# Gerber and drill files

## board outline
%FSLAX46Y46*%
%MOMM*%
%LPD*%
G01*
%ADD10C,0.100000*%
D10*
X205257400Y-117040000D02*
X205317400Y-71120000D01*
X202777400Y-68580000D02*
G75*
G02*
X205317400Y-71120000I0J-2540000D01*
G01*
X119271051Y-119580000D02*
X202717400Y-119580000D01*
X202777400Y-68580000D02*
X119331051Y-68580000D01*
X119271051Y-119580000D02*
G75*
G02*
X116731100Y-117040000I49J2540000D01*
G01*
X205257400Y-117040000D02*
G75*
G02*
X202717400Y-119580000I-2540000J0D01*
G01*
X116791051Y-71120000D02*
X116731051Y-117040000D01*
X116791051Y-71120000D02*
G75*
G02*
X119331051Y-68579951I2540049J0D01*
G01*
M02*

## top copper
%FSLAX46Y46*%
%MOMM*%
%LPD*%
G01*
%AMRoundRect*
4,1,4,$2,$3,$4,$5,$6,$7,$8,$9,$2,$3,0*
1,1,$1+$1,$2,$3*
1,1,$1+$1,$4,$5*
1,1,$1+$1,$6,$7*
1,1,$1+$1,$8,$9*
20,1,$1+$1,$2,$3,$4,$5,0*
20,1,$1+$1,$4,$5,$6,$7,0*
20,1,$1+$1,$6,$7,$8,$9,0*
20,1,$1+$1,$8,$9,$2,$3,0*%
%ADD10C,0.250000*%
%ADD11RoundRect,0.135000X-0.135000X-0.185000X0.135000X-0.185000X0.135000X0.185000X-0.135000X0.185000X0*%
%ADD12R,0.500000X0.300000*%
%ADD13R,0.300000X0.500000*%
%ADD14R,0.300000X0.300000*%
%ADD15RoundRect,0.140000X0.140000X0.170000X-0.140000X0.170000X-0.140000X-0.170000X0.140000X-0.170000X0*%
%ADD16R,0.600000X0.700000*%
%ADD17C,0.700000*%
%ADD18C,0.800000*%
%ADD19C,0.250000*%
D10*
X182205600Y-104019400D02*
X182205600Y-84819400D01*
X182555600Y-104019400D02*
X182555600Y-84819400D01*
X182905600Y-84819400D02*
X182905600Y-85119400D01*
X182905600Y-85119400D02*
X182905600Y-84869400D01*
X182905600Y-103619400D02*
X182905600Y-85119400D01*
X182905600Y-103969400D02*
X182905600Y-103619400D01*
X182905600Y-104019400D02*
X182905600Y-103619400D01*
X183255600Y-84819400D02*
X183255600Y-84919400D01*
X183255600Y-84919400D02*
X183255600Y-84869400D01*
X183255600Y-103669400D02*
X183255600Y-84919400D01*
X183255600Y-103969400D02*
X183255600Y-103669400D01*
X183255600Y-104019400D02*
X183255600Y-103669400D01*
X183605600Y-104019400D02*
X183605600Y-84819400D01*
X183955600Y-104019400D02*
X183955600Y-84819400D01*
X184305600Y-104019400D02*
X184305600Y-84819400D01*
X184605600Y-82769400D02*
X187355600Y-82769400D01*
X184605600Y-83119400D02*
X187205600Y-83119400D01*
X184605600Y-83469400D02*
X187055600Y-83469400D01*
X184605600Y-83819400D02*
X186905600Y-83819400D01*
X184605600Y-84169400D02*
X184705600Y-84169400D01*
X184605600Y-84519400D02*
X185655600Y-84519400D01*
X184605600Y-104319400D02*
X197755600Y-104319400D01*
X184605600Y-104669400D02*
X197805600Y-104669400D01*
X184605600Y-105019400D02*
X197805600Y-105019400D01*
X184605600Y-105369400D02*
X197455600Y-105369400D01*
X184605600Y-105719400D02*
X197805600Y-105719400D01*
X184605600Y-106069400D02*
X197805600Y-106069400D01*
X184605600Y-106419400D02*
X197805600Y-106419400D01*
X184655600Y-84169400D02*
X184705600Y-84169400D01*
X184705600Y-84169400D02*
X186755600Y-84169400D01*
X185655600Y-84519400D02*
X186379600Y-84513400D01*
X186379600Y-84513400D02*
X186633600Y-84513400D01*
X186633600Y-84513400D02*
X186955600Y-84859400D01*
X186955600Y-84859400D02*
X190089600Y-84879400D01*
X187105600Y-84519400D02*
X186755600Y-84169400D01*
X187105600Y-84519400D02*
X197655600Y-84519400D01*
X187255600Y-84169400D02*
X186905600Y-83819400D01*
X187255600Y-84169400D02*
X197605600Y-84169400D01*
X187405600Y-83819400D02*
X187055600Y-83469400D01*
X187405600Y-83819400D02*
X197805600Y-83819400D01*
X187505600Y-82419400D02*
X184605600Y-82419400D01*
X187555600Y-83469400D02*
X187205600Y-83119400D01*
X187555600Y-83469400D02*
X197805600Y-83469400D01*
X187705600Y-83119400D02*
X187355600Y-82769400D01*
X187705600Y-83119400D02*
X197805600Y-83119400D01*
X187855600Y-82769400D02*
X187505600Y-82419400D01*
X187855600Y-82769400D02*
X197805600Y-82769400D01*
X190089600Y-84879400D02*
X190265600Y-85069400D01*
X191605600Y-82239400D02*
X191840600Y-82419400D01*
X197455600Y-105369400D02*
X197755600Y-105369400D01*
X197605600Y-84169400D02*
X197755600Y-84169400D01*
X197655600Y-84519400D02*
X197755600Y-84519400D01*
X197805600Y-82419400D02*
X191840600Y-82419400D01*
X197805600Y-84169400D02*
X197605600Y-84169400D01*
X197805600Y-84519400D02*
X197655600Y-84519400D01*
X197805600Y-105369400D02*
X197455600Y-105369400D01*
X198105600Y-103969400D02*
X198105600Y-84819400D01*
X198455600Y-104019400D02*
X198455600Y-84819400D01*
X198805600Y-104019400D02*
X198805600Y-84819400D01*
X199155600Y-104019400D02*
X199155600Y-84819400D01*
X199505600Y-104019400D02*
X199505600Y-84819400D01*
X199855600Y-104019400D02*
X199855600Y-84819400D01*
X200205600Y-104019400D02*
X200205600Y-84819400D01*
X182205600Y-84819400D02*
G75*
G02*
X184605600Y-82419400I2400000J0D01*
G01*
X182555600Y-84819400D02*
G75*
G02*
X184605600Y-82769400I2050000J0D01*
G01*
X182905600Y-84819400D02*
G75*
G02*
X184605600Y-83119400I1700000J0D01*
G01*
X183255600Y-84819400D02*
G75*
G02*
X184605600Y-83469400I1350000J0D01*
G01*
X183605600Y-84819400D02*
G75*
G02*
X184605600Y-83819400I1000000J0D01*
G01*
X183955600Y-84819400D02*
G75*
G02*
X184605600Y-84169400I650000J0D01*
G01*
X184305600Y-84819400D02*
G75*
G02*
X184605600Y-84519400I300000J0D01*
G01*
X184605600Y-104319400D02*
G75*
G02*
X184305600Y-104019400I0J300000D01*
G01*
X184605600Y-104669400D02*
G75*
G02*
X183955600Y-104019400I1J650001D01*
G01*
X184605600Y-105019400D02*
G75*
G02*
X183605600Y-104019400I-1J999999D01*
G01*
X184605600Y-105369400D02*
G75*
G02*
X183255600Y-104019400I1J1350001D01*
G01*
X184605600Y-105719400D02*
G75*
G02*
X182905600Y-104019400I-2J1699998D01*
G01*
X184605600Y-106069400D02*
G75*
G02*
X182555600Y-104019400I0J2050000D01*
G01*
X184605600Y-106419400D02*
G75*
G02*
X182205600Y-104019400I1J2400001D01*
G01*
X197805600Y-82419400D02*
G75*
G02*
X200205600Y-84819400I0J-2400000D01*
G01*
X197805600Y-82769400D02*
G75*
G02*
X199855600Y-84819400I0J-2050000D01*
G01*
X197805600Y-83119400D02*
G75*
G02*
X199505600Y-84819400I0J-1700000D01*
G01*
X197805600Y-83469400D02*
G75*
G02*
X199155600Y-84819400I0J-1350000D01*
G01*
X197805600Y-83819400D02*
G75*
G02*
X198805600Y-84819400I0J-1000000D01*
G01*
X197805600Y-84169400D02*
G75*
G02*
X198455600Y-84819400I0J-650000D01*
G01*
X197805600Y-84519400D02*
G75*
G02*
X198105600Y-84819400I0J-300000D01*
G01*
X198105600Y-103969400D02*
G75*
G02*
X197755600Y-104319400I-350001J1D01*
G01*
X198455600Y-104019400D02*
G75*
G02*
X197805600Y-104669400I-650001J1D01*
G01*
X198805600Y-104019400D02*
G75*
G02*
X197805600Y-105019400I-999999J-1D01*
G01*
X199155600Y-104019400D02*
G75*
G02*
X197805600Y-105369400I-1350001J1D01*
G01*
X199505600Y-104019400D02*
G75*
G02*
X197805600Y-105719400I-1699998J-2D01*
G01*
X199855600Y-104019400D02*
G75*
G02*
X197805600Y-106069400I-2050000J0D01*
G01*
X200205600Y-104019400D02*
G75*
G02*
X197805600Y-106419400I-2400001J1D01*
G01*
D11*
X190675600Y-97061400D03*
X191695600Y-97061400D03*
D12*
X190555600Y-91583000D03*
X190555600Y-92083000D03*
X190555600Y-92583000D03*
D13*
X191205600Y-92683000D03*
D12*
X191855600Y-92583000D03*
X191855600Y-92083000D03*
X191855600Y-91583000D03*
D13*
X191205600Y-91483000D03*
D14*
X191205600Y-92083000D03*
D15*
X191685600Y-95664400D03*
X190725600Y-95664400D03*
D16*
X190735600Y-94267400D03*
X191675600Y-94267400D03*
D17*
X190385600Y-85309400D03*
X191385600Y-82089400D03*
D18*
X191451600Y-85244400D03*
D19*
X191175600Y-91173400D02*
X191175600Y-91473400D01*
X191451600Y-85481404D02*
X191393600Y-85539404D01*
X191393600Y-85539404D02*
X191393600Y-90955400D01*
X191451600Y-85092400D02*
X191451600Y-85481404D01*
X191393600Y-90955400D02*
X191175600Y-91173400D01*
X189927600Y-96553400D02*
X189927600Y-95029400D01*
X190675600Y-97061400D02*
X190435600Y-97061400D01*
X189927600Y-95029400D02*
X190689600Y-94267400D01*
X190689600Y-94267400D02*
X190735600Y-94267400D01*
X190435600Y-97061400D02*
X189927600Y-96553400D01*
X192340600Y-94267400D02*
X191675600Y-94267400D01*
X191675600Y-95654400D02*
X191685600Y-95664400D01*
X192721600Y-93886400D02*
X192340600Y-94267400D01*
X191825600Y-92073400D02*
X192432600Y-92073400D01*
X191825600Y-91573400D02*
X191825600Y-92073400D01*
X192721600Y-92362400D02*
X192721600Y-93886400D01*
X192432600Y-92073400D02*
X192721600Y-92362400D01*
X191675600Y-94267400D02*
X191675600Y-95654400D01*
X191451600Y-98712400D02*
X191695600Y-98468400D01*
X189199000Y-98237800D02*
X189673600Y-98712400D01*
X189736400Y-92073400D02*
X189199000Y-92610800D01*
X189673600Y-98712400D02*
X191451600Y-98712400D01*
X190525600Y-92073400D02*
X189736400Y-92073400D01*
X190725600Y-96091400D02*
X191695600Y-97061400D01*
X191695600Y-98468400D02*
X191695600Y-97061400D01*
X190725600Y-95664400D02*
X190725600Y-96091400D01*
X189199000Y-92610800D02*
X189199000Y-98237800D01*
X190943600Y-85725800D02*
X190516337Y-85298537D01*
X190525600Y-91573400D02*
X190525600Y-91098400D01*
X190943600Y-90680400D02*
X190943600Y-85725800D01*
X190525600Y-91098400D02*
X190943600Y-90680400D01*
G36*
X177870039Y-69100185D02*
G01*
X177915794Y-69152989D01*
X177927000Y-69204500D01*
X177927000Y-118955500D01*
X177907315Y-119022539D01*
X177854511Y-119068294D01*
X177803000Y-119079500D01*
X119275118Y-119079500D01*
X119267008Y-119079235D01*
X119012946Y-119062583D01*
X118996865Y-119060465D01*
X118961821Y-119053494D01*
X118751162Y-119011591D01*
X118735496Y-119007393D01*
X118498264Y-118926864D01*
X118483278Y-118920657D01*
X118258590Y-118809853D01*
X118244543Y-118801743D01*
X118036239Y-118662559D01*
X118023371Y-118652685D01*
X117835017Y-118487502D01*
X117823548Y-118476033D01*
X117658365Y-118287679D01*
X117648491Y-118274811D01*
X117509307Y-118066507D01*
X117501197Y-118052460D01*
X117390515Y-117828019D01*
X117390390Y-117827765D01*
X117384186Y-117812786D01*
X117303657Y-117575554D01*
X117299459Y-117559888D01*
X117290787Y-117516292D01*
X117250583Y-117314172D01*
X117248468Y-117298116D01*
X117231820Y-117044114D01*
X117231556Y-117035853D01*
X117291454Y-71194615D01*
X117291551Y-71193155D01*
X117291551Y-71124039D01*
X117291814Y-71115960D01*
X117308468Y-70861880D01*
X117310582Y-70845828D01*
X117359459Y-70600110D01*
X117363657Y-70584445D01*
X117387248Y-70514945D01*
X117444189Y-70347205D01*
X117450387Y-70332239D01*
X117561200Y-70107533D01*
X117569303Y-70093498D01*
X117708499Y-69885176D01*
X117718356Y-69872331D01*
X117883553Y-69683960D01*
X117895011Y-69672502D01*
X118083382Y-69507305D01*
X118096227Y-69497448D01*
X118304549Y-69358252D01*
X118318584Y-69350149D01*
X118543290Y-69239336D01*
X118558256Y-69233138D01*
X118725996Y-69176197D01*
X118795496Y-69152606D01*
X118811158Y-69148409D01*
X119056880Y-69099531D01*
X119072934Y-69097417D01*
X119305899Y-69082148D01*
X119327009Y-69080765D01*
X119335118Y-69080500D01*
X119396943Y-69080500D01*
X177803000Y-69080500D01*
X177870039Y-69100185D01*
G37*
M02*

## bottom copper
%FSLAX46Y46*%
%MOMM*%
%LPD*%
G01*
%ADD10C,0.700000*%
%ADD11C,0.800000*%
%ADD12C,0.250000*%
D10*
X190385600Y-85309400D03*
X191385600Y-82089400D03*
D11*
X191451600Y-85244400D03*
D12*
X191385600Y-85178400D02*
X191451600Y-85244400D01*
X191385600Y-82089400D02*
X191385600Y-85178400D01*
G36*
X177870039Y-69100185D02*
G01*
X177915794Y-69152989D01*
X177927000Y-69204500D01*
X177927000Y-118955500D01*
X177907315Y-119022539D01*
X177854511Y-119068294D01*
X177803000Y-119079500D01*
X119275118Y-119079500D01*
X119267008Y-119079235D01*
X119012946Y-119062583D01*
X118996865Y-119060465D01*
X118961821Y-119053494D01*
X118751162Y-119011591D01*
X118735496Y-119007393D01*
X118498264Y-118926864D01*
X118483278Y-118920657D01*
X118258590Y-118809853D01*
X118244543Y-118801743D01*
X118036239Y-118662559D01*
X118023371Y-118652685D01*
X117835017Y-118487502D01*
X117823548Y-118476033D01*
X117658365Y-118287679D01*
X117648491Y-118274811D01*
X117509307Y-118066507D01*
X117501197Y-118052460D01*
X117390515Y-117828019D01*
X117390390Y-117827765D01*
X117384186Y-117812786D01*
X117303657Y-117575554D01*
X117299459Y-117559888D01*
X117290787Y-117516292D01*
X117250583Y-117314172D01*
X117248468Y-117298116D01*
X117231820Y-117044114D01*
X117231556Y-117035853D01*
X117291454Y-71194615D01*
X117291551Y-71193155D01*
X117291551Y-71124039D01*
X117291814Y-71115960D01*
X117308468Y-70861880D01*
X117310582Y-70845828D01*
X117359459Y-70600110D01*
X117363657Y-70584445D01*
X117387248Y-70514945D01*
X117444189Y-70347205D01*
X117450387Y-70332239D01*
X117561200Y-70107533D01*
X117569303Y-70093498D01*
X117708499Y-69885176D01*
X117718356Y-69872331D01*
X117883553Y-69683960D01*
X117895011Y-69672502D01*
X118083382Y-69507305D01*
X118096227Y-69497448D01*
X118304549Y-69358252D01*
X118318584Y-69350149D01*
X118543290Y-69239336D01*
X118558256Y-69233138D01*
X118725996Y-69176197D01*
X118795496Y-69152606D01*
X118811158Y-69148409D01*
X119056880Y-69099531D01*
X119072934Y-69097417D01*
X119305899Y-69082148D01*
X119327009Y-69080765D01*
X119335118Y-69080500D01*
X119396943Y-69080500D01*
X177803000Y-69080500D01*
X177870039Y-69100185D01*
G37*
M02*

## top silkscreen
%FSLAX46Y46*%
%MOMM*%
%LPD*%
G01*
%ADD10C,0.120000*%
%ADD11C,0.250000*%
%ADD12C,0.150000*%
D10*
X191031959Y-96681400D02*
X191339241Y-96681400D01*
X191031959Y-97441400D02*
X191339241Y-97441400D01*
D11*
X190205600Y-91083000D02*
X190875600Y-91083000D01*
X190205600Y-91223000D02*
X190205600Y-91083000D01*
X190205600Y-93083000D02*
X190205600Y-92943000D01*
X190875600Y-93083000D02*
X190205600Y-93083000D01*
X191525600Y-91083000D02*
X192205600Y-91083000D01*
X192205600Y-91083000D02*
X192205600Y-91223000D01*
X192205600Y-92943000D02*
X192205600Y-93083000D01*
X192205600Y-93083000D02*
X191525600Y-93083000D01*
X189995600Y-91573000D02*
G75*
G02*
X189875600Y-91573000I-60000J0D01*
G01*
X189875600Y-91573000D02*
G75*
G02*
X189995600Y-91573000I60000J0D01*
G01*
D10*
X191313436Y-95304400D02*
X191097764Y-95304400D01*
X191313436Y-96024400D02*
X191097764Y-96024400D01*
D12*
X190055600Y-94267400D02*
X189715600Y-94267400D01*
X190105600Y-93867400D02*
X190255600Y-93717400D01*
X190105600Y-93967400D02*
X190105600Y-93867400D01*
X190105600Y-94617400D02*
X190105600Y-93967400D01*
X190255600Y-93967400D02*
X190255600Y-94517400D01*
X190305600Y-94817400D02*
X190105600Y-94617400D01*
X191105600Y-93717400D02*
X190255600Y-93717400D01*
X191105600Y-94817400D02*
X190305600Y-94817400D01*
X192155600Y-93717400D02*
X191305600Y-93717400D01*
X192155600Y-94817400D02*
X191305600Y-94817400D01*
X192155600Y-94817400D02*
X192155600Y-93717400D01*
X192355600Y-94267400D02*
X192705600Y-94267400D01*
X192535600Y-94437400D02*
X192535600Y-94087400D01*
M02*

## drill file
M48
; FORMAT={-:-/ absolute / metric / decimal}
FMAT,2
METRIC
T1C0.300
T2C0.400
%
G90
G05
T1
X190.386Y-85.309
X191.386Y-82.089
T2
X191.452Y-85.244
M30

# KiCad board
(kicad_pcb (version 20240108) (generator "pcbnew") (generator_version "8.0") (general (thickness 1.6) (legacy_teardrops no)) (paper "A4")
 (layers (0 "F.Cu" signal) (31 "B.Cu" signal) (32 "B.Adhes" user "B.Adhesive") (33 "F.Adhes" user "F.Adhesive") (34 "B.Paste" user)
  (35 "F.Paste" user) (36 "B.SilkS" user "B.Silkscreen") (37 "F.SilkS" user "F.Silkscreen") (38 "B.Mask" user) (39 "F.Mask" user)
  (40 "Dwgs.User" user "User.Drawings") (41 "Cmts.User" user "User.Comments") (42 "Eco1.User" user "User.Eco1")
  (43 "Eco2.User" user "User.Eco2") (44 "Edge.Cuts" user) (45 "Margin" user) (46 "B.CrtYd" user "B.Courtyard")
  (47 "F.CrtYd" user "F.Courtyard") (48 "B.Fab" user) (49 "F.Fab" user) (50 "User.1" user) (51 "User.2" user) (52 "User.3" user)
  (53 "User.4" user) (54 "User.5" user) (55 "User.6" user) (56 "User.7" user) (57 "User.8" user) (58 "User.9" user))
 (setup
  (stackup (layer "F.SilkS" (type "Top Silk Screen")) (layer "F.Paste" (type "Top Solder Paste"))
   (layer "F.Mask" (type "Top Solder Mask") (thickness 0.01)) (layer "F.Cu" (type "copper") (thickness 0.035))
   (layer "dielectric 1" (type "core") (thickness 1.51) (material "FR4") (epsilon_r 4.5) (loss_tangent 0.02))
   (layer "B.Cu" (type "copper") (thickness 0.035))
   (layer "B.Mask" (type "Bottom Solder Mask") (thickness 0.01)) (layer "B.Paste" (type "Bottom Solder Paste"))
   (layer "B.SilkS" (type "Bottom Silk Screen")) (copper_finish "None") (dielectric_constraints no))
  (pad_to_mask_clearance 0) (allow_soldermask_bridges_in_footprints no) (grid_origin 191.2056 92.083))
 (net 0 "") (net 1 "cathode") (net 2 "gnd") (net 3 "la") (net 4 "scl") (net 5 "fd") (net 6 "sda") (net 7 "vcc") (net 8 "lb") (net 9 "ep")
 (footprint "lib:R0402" (layer "F.Cu") (at 191.1856 97.0614)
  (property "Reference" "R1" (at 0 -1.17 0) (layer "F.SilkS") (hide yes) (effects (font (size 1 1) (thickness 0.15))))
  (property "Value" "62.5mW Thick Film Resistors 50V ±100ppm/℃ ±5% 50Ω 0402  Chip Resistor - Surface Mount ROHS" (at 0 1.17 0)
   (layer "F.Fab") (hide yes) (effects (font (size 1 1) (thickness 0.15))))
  (fp_line (start -0.153641 -0.38) (end 0.153641 -0.38) (stroke (width 0.12) (type solid)) (layer "F.SilkS"))
  (fp_line (start -0.153641 0.38) (end 0.153641 0.38) (stroke (width 0.12) (type solid)) (layer "F.SilkS"))
  (pad "1" smd roundrect (at -0.51 0) (size 0.54 0.64) (layers "F.Cu" "F.Paste" "F.Mask") (roundrect_rratio 0.25) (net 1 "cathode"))
  (pad "2" smd roundrect (at 0.51 0) (size 0.54 0.64) (layers "F.Cu" "F.Paste" "F.Mask") (roundrect_rratio 0.25) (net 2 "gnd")))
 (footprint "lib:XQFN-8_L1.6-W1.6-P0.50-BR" (layer "F.Cu") (at 191.2056 92.083 180)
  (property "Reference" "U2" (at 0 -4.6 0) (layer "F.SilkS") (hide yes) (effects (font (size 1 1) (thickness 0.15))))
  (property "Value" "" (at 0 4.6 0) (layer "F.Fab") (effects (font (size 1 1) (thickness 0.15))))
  (fp_line (start 1 1) (end 0.33 1) (stroke (width 0.25) (type solid)) (layer "F.SilkS"))
  (fp_line (start 1 0.86) (end 1 1) (stroke (width 0.25) (type solid)) (layer "F.SilkS"))
  (fp_line (start 1 -1) (end 1 -0.86) (stroke (width 0.25) (type solid)) (layer "F.SilkS"))
  (fp_line (start 0.33 -1) (end 1 -1) (stroke (width 0.25) (type solid)) (layer "F.SilkS"))
  (fp_line (start -0.32 1) (end -1 1) (stroke (width 0.25) (type solid)) (layer "F.SilkS"))
  (fp_line (start -1 1) (end -1 0.86) (stroke (width 0.25) (type solid)) (layer "F.SilkS"))
  (fp_line (start -1 -0.86) (end -1 -1) (stroke (width 0.25) (type solid)) (layer "F.SilkS"))
  (fp_line (start -1 -1) (end -0.32 -1) (stroke (width 0.25) (type solid)) (layer "F.SilkS"))
  (fp_circle (center 1.27 0.51) (end 1.33 0.51) (stroke (width 0.25) (type solid)) (fill none) (layer "F.SilkS"))
  (pad "1" smd rect (at 0.65 0.5) (size 0.5 0.3) (layers "F.Cu" "F.Paste" "F.Mask") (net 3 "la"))
  (pad "2" smd rect (at 0.65 0) (size 0.5 0.3) (layers "F.Cu" "F.Paste" "F.Mask") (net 2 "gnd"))
  (pad "3" smd rect (at 0.65 -0.5) (size 0.5 0.3) (layers "F.Cu" "F.Paste" "F.Mask") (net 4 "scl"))
  (pad "4" smd rect (at 0 -0.6 90) (size 0.5 0.3) (layers "F.Cu" "F.Paste" "F.Mask") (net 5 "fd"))
  (pad "5" smd rect (at -0.65 -0.5) (size 0.5 0.3) (layers "F.Cu" "F.Paste" "F.Mask") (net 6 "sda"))
  (pad "6" smd rect (at -0.65 0) (size 0.5 0.3) (layers "F.Cu" "F.Paste" "F.Mask") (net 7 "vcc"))
  (pad "7" smd rect (at -0.65 0.5) (size 0.5 0.3) (layers "F.Cu" "F.Paste" "F.Mask") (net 7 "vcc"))
  (pad "8" smd rect (at 0 0.6 90) (size 0.5 0.3) (layers "F.Cu" "F.Paste" "F.Mask") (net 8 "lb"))
  (pad "9" smd rect (at 0 0 90) (size 0.3 0.3) (layers "F.Cu" "F.Paste" "F.Mask") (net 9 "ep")))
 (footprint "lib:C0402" (layer "F.Cu") (at 191.2056 95.6644 180)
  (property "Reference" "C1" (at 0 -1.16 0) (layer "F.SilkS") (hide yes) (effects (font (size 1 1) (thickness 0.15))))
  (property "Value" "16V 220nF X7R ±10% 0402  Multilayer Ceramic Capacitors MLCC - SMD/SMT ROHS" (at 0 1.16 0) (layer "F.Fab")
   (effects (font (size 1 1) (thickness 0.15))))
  (fp_line (start -0.107836 0.36) (end 0.107836 0.36) (stroke (width 0.12) (type solid)) (layer "F.SilkS"))
  (fp_line (start -0.107836 -0.36) (end 0.107836 -0.36) (stroke (width 0.12) (type solid)) (layer "F.SilkS"))
  (pad "1" smd roundrect (at -0.48 0 180) (size 0.56 0.62) (layers "F.Cu" "F.Paste" "F.Mask") (roundrect_rratio 0.25) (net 7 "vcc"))
  (pad "2" smd roundrect (at 0.48 0 180) (size 0.56 0.62) (layers "F.Cu" "F.Paste" "F.Mask") (roundrect_rratio 0.25) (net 2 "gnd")))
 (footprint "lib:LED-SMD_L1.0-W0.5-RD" (layer "F.Cu") (at 191.2056 94.2674)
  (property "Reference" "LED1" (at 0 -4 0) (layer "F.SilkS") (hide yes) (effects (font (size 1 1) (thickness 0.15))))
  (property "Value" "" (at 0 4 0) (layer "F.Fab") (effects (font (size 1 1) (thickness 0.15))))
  (fp_line (start -1.15 0) (end -1.49 0) (stroke (width 0.15) (type solid)) (layer "F.SilkS"))
  (fp_line (start -1.1 -0.4) (end -0.95 -0.55) (stroke (width 0.15) (type solid)) (layer "F.SilkS"))
  (fp_line (start -1.1 -0.3) (end -1.1 -0.4) (stroke (width 0.15) (type solid)) (layer "F.SilkS"))
  (fp_line (start -1.1 0.35) (end -1.1 -0.3) (stroke (width 0.15) (type solid)) (layer "F.SilkS"))
  (fp_line (start -0.95 -0.3) (end -0.95 0.25) (stroke (width 0.15) (type solid)) (layer "F.SilkS"))
  (fp_line (start -0.9 0.55) (end -1.1 0.35) (stroke (width 0.15) (type solid)) (layer "F.SilkS"))
  (fp_line (start -0.1 -0.55) (end -0.95 -0.55) (stroke (width 0.15) (type solid)) (layer "F.SilkS"))
  (fp_line (start -0.1 0.55) (end -0.9 0.55) (stroke (width 0.15) (type solid)) (layer "F.SilkS"))
  (fp_line (start 0.95 -0.55) (end 0.1 -0.55) (stroke (width 0.15) (type solid)) (layer "F.SilkS"))
  (fp_line (start 0.95 0.55) (end 0.1 0.55) (stroke (width 0.15) (type solid)) (layer "F.SilkS"))
  (fp_line (start 0.95 0.55) (end 0.95 -0.55) (stroke (width 0.15) (type solid)) (layer "F.SilkS"))
  (fp_line (start 1.15 0) (end 1.5 0) (stroke (width 0.15) (type solid)) (layer "F.SilkS"))
  (fp_line (start 1.33 0.17) (end 1.33 -0.18) (stroke (width 0.15) (type solid)) (layer "F.SilkS"))
  (pad "1" smd rect (at -0.47 0 180) (size 0.6 0.7) (layers "F.Cu" "F.Paste" "F.Mask") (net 1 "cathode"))
  (pad "2" smd rect (at 0.47 0 180) (size 0.6 0.7) (layers "F.Cu" "F.Paste" "F.Mask") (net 7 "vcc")))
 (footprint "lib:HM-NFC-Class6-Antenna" (layer "F.Cu") (at 191.2056 94.4194 90)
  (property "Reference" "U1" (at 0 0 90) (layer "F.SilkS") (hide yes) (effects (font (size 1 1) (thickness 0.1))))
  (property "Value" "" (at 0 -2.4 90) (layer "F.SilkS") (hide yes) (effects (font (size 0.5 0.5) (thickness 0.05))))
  (fp_line (start -9.6 -9) (end 9.6 -9) (stroke (width 0.25) (type solid)) (layer "F.Cu"))
  (fp_line (start -9.6 -8.65) (end 9.6 -8.65) (stroke (width 0.25) (type solid)) (layer "F.Cu"))
  (fp_line (start 9.6 -8.3) (end 9.3 -8.3) (stroke (width 0.25) (type solid)) (layer "F.Cu"))
  (fp_line (start 9.3 -8.3) (end 9.55 -8.3) (stroke (width 0.25) (type solid)) (layer "F.Cu"))
  (fp_line (start -9.2 -8.3) (end 9.3 -8.3) (stroke (width 0.25) (type solid)) (layer "F.Cu"))
  (fp_line (start -9.55 -8.3) (end -9.2 -8.3) (stroke (width 0.25) (type solid)) (layer "F.Cu"))
  (fp_line (start -9.6 -8.3) (end -9.2 -8.3) (stroke (width 0.25) (type solid)) (layer "F.Cu"))
  (fp_line (start 9.6 -7.95) (end 9.5 -7.95) (stroke (width 0.25) (type solid)) (layer "F.Cu"))
  (fp_line (start 9.5 -7.95) (end 9.55 -7.95) (stroke (width 0.25) (type solid)) (layer "F.Cu"))
  (fp_line (start -9.25 -7.95) (end 9.5 -7.95) (stroke (width 0.25) (type solid)) (layer "F.Cu"))
  (fp_line (start -9.55 -7.95) (end -9.25 -7.95) (stroke (width 0.25) (type solid)) (layer "F.Cu"))
  (fp_line (start -9.6 -7.95) (end -9.25 -7.95) (stroke (width 0.25) (type solid)) (layer "F.Cu"))
  (fp_line (start -9.6 -7.6) (end 9.6 -7.6) (stroke (width 0.25) (type solid)) (layer "F.Cu"))
  (fp_line (start -9.6 -7.25) (end 9.6 -7.25) (stroke (width 0.25) (type solid)) (layer "F.Cu"))
  (fp_line (start -9.6 -6.9) (end 9.6 -6.9) (stroke (width 0.25) (type solid)) (layer "F.Cu"))
  (fp_line (start 11.65 -6.6) (end 11.65 -3.85) (stroke (width 0.25) (type solid)) (layer "F.Cu"))
  (fp_line (start 11.3 -6.6) (end 11.3 -4) (stroke (width 0.25) (type solid)) (layer "F.Cu"))
  (fp_line (start 10.95 -6.6) (end 10.95 -4.15) (stroke (width 0.25) (type solid)) (layer "F.Cu"))
  (fp_line (start 10.6 -6.6) (end 10.6 -4.3) (stroke (width 0.25) (type solid)) (layer "F.Cu"))
  (fp_line (start 10.25 -6.6) (end 10.25 -6.5) (stroke (width 0.25) (type solid)) (layer "F.Cu"))
  (fp_line (start 9.9 -6.6) (end 9.9 -5.55) (stroke (width 0.25) (type solid)) (layer "F.Cu"))
  (fp_line (start -9.9 -6.6) (end -9.9 6.55) (stroke (width 0.25) (type solid)) (layer "F.Cu"))
  (fp_line (start -10.25 -6.6) (end -10.25 6.6) (stroke (width 0.25) (type solid)) (layer "F.Cu"))
  (fp_line (start -10.6 -6.6) (end -10.6 6.6) (stroke (width 0.25) (type solid)) (layer "F.Cu"))
  (fp_line (start -10.95 -6.6) (end -10.95 6.25) (stroke (width 0.25) (type solid)) (layer "F.Cu"))
  (fp_line (start -11.3 -6.6) (end -11.3 6.6) (stroke (width 0.25) (type solid)) (layer "F.Cu"))
  (fp_line (start -11.65 -6.6) (end -11.65 6.6) (stroke (width 0.25) (type solid)) (layer "F.Cu"))
  (fp_line (start -12 -6.6) (end -12 6.6) (stroke (width 0.25) (type solid)) (layer "F.Cu"))
  (fp_line (start 10.25 -6.55) (end 10.25 -6.5) (stroke (width 0.25) (type solid)) (layer "F.Cu"))
  (fp_line (start 10.25 -6.5) (end 10.25 -4.45) (stroke (width 0.25) (type solid)) (layer "F.Cu"))
  (fp_line (start 9.9 -5.55) (end 9.906 -4.826) (stroke (width 0.25) (type solid)) (layer "F.Cu"))
  (fp_line (start 9.906 -4.826) (end 9.906 -4.572) (stroke (width 0.25) (type solid)) (layer "F.Cu"))
  (fp_line (start 9.906 -4.572) (end 9.56 -4.25) (stroke (width 0.25) (type solid)) (layer "F.Cu"))
  (fp_line (start 9.56 -4.25) (end 9.54 -1.116) (stroke (width 0.25) (type solid)) (layer "F.Cu"))
  (fp_line (start 9.9 -4.1) (end 10.25 -4.45) (stroke (width 0.25) (type solid)) (layer "F.Cu"))
  (fp_line (start 9.9 -4.1) (end 9.9 6.45) (stroke (width 0.25) (type solid)) (layer "F.Cu"))
  (fp_line (start 10.25 -3.95) (end 10.6 -4.3) (stroke (width 0.25) (type solid)) (layer "F.Cu"))
  (fp_line (start 10.25 -3.95) (end 10.25 6.4) (stroke (width 0.25) (type solid)) (layer "F.Cu"))
  (fp_line (start 10.6 -3.8) (end 10.95 -4.15) (stroke (width 0.25) (type solid)) (layer "F.Cu"))
  (fp_line (start 10.6 -3.8) (end 10.6 6.6) (stroke (width 0.25) (type solid)) (layer "F.Cu"))
  (fp_line (start 12 -3.7) (end 12 -6.6) (stroke (width 0.25) (type solid)) (layer "F.Cu"))
  (fp_line (start 10.95 -3.65) (end 11.3 -4) (stroke (width 0.25) (type solid)) (layer "F.Cu"))
  (fp_line (start 10.95 -3.65) (end 10.95 6.6) (stroke (width 0.25) (type solid)) (layer "F.Cu"))
  (fp_line (start 11.3 -3.5) (end 11.65 -3.85) (stroke (width 0.25) (type solid)) (layer "F.Cu"))
  (fp_line (start 11.3 -3.5) (end 11.3 6.6) (stroke (width 0.25) (type solid)) (layer "F.Cu"))
  (fp_line (start 11.65 -3.35) (end 12 -3.7) (stroke (width 0.25) (type solid)) (layer "F.Cu"))
  (fp_line (start 11.65 -3.35) (end 11.65 6.6) (stroke (width 0.25) (type solid)) (layer "F.Cu"))
  (fp_line (start 9.54 -1.116) (end 9.35 -0.94) (stroke (width 0.25) (type default)) (layer "F.Cu"))
  (fp_line (start 12.18 0.4) (end 12 0.635) (stroke (width 0.25) (type default)) (layer "F.Cu"))
  (fp_line (start -10.95 6.25) (end -10.95 6.55) (stroke (width 0.25) (type solid)) (layer "F.Cu"))
  (fp_line (start 10.25 6.4) (end 10.25 6.55) (stroke (width 0.25) (type solid)) (layer "F.Cu"))
  (fp_line (start 9.9 6.45) (end 9.9 6.55) (stroke (width 0.25) (type solid)) (layer "F.Cu"))
  (fp_line (start 12 6.6) (end 12 0.635) (stroke (width 0.25) (type solid)) (layer "F.Cu"))
  (fp_line (start 10.25 6.6) (end 10.25 6.4) (stroke (width 0.25) (type solid)) (layer "F.Cu"))
  (fp_line (start 9.9 6.6) (end 9.9 6.45) (stroke (width 0.25) (type solid)) (layer "F.Cu"))
  (fp_line (start -10.95 6.6) (end -10.95 6.25) (stroke (width 0.25) (type solid)) (layer "F.Cu"))
  (fp_line (start -9.55 6.9) (end 9.6 6.9) (stroke (width 0.25) (type solid)) (layer "F.Cu"))
  (fp_line (start -9.6 7.25) (end 9.6 7.25) (stroke (width 0.25) (type solid)) (layer "F.Cu"))
  (fp_line (start -9.6 7.6) (end 9.6 7.6) (stroke (width 0.25) (type solid)) (layer "F.Cu"))
  (fp_line (start -9.6 7.95) (end 9.6 7.95) (stroke (width 0.25) (type solid)) (layer "F.Cu"))
  (fp_line (start -9.6 8.3) (end 9.6 8.3) (stroke (width 0.25) (type solid)) (layer "F.Cu"))
  (fp_line (start -9.6 8.65) (end 9.6 8.65) (stroke (width 0.25) (type solid)) (layer "F.Cu"))
  (fp_line (start -9.6 9) (end 9.6 9) (stroke (width 0.25) (type solid)) (layer "F.Cu"))
  (fp_arc (start 9.6 -9) (mid 11.297056 -8.297056) (end 12 -6.6) (stroke (width 0.25) (type solid)) (layer "F.Cu"))
  (fp_arc (start 9.6 -8.65) (mid 11.049569 -8.049569) (end 11.65 -6.6) (stroke (width 0.25) (type solid)) (layer "F.Cu"))
  (fp_arc (start 9.6 -8.3) (mid 10.802082 -7.802082) (end 11.3 -6.6) (stroke (width 0.25) (type solid)) (layer "F.Cu"))
  (fp_arc (start 9.6 -7.95) (mid 10.554594 -7.554594) (end 10.95 -6.6) (stroke (width 0.25) (type solid)) (layer "F.Cu"))
  (fp_arc (start 9.6 -7.6) (mid 10.307107 -7.307107) (end 10.6 -6.6) (stroke (width 0.25) (type solid)) (layer "F.Cu"))
  (fp_arc (start 9.6 -7.25) (mid 10.059619 -7.059619) (end 10.25 -6.6) (stroke (width 0.25) (type solid)) (layer "F.Cu"))
  (fp_arc (start 9.6 -6.9) (mid 9.812132 -6.812132) (end 9.9 -6.6) (stroke (width 0.25) (type solid)) (layer "F.Cu"))
  (fp_arc (start -9.9 -6.6) (mid -9.812132 -6.812132) (end -9.6 -6.9) (stroke (width 0.25) (type solid)) (layer "F.Cu"))
  (fp_arc (start -10.25 -6.6) (mid -10.059619 -7.059619) (end -9.6 -7.25) (stroke (width 0.25) (type solid)) (layer "F.Cu"))
  (fp_arc (start -10.6 -6.6) (mid -10.307107 -7.307107) (end -9.6 -7.6) (stroke (width 0.25) (type solid)) (layer "F.Cu"))
  (fp_arc (start -10.95 -6.6) (mid -10.554594 -7.554594) (end -9.6 -7.95) (stroke (width 0.25) (type solid)) (layer "F.Cu"))
  (fp_arc (start -11.3 -6.6) (mid -10.802082 -7.802082) (end -9.6 -8.3) (stroke (width 0.25) (type solid)) (layer "F.Cu"))
  (fp_arc (start -11.65 -6.6) (mid -11.049569 -8.049569) (end -9.6 -8.65) (stroke (width 0.25) (type solid)) (layer "F.Cu"))
  (fp_arc (start -12 -6.6) (mid -11.297056 -8.297056) (end -9.6 -9) (stroke (width 0.25) (type solid)) (layer "F.Cu"))
  (fp_arc (start 12 6.6) (mid 11.297056 8.297056) (end 9.6 9) (stroke (width 0.25) (type solid)) (layer "F.Cu"))
  (fp_arc (start 11.65 6.6) (mid 11.049569 8.049569) (end 9.6 8.65) (stroke (width 0.25) (type solid)) (layer "F.Cu"))
  (fp_arc (start 11.3 6.6) (mid 10.802082 7.802082) (end 9.6 8.3) (stroke (width 0.25) (type solid)) (layer "F.Cu"))
  (fp_arc (start 10.95 6.6) (mid 10.554594 7.554594) (end 9.6 7.95) (stroke (width 0.25) (type solid)) (layer "F.Cu"))
  (fp_arc (start 10.6 6.6) (mid 10.307107 7.307107) (end 9.6 7.6) (stroke (width 0.25) (type solid)) (layer "F.Cu"))
  (fp_arc (start 10.25 6.6) (mid 10.059619 7.059619) (end 9.6 7.25) (stroke (width 0.25) (type solid)) (layer "F.Cu"))
  (fp_arc (start 9.9 6.6) (mid 9.812132 6.812132) (end 9.6 6.9) (stroke (width 0.25) (type solid)) (layer "F.Cu"))
  (fp_arc (start -9.55 6.9) (mid -9.797487 6.797487) (end -9.9 6.55) (stroke (width 0.25) (type solid)) (layer "F.Cu"))
  (fp_arc (start -9.6 7.25) (mid -10.059619 7.059619) (end -10.25 6.6) (stroke (width 0.25) (type solid)) (layer "F.Cu"))
  (fp_arc (start -9.6 7.6) (mid -10.307107 7.307107) (end -10.6 6.6) (stroke (width 0.25) (type solid)) (layer "F.Cu"))
  (fp_arc (start -9.6 7.95) (mid -10.554594 7.554594) (end -10.95 6.6) (stroke (width 0.25) (type solid)) (layer "F.Cu"))
  (fp_arc (start -9.6 8.3) (mid -10.802082 7.802082) (end -11.3 6.6) (stroke (width 0.25) (type solid)) (layer "F.Cu"))
  (fp_arc (start -9.6 8.65) (mid -11.049569 8.049569) (end -11.65 6.6) (stroke (width 0.25) (type solid)) (layer "F.Cu"))
  (fp_arc (start -9.6 9) (mid -11.297056 8.297056) (end -12 6.6) (stroke (width 0.25) (type solid)) (layer "F.Cu"))
  (pad "1" thru_hole circle (at 9.11 -0.82 90) (size 0.7 0.7) (drill 0.3) (layers "*.Cu" "*.Mask") (remove_unused_layers no) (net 3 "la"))
  (pad "2" thru_hole circle (at 12.33 0.18 90) (size 0.7 0.7) (drill 0.3) (layers "*.Cu" "*.Mask") (remove_unused_layers no) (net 8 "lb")))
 (gr_line (start 205.2574 117.04) (end 205.3174 71.12) (stroke (width 0.1) (type default)) (layer "Edge.Cuts"))
 (gr_arc (start 202.7774 68.58) (mid 204.573451 69.323949) (end 205.3174 71.12) (stroke (width 0.1) (type default)) (layer "Edge.Cuts"))
 (gr_line (start 119.271051 119.58) (end 202.7174 119.58) (stroke (width 0.1) (type default)) (layer "Edge.Cuts"))
 (gr_line (start 202.7774 68.58) (end 119.331051 68.58) (stroke (width 0.1) (type default)) (layer "Edge.Cuts"))
 (gr_arc (start 119.271051 119.58) (mid 117.475 118.836051) (end 116.731051 117.04) (stroke (width 0.1) (type default)) (layer "Edge.Cuts"))
 (gr_arc (start 205.2574 117.04) (mid 204.513451 118.836051) (end 202.7174 119.58) (stroke (width 0.1) (type default)) (layer "Edge.Cuts"))
 (gr_line (start 116.791051 71.12) (end 116.731051 117.04) (stroke (width 0.1) (type default)) (layer "Edge.Cuts"))
 (gr_arc (start 116.791051 71.12) (mid 117.535 69.323949) (end 119.331051 68.58) (stroke (width 0.1) (type default)) (layer "Edge.Cuts"))
 (segment (start 191.1756 91.1734) (end 191.1756 91.4734) (width 0.25) (layer "F.Cu") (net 8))
 (segment (start 191.4516 85.481404) (end 191.3936 85.539404) (width 0.25) (layer "F.Cu") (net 8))
 (segment (start 191.3936 85.539404) (end 191.3936 90.9554) (width 0.25) (layer "F.Cu") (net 8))
 (segment (start 191.4516 85.0924) (end 191.4516 85.481404) (width 0.25) (layer "F.Cu") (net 8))
 (segment (start 191.3936 90.9554) (end 191.1756 91.1734) (width 0.25) (layer "F.Cu") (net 8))
 (via (at 191.4516 85.2444) (size 0.8) (drill 0.4) (layers "F.Cu" "B.Cu") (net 8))
 (segment (start 191.3856 85.1784) (end 191.4516 85.2444) (width 0.25) (layer "B.Cu") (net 8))
 (segment (start 191.3856 82.0894) (end 191.3856 85.1784) (width 0.25) (layer "B.Cu") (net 8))
 (segment (start 189.9276 96.5534) (end 189.9276 95.0294) (width 0.25) (layer "F.Cu") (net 1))
 (segment (start 190.6756 97.0614) (end 190.4356 97.0614) (width 0.25) (layer "F.Cu") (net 1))
 (segment (start 189.9276 95.0294) (end 190.6896 94.2674) (width 0.25) (layer "F.Cu") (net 1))
 (segment (start 190.6896 94.2674) (end 190.7356 94.2674) (width 0.25) (layer "F.Cu") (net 1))
 (segment (start 190.4356 97.0614) (end 189.9276 96.5534) (width 0.25) (layer "F.Cu") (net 1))
 (segment (start 192.3406 94.2674) (end 191.6756 94.2674) (width 0.25) (layer "F.Cu") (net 7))
 (segment (start 191.6756 95.6544) (end 191.6856 95.6644) (width 0.25) (layer "F.Cu") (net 7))
 (segment (start 192.7216 93.8864) (end 192.3406 94.2674) (width 0.25) (layer "F.Cu") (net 7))
 (segment (start 191.8256 92.0734) (end 192.4326 92.0734) (width 0.25) (layer "F.Cu") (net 7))
 (segment (start 191.8256 91.5734) (end 191.8256 92.0734) (width 0.25) (layer "F.Cu") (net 7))
 (segment (start 192.7216 92.3624) (end 192.7216 93.8864) (width 0.25) (layer "F.Cu") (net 7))
 (segment (start 192.4326 92.0734) (end 192.7216 92.3624) (width 0.25) (layer "F.Cu") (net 7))
 (segment (start 191.6756 94.2674) (end 191.6756 95.6544) (width 0.25) (layer "F.Cu") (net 7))
 (segment (start 191.4516 98.7124) (end 191.6956 98.4684) (width 0.25) (layer "F.Cu") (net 2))
 (segment (start 189.199 98.2378) (end 189.6736 98.7124) (width 0.25) (layer "F.Cu") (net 2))
 (segment (start 189.7364 92.0734) (end 189.199 92.6108) (width 0.25) (layer "F.Cu") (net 2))
 (segment (start 189.6736 98.7124) (end 191.4516 98.7124) (width 0.25) (layer "F.Cu") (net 2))
 (segment (start 190.5256 92.0734) (end 189.7364 92.0734) (width 0.25) (layer "F.Cu") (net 2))
 (segment (start 190.7256 96.0914) (end 191.6956 97.0614) (width 0.25) (layer "F.Cu") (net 2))
 (segment (start 191.6956 98.4684) (end 191.6956 97.0614) (width 0.25) (layer "F.Cu") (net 2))
 (segment (start 190.7256 95.6644) (end 190.7256 96.0914) (width 0.25) (layer "F.Cu") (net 2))
 (segment (start 189.199 92.6108) (end 189.199 98.2378) (width 0.25) (layer "F.Cu") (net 2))
 (segment (start 190.9436 85.7258) (end 190.516337 85.298537) (width 0.25) (layer "F.Cu") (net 3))
 (segment (start 190.5256 91.5734) (end 190.5256 91.0984) (width 0.25) (layer "F.Cu") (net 3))
 (segment (start 190.9436 90.6804) (end 190.9436 85.7258) (width 0.25) (layer "F.Cu") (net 3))
 (segment (start 190.5256 91.0984) (end 190.9436 90.6804) (width 0.25) (layer "F.Cu") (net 3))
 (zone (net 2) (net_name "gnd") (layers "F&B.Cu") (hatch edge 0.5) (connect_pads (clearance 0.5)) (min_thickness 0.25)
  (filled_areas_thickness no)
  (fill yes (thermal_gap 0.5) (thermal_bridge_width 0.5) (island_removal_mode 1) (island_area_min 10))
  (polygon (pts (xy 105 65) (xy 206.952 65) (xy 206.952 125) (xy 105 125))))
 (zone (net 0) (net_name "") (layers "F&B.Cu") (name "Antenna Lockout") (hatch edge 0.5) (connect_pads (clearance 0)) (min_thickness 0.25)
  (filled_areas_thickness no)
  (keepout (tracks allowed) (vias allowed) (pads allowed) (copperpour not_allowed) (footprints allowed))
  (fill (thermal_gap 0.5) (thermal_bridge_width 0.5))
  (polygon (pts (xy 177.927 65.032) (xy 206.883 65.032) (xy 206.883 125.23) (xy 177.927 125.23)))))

